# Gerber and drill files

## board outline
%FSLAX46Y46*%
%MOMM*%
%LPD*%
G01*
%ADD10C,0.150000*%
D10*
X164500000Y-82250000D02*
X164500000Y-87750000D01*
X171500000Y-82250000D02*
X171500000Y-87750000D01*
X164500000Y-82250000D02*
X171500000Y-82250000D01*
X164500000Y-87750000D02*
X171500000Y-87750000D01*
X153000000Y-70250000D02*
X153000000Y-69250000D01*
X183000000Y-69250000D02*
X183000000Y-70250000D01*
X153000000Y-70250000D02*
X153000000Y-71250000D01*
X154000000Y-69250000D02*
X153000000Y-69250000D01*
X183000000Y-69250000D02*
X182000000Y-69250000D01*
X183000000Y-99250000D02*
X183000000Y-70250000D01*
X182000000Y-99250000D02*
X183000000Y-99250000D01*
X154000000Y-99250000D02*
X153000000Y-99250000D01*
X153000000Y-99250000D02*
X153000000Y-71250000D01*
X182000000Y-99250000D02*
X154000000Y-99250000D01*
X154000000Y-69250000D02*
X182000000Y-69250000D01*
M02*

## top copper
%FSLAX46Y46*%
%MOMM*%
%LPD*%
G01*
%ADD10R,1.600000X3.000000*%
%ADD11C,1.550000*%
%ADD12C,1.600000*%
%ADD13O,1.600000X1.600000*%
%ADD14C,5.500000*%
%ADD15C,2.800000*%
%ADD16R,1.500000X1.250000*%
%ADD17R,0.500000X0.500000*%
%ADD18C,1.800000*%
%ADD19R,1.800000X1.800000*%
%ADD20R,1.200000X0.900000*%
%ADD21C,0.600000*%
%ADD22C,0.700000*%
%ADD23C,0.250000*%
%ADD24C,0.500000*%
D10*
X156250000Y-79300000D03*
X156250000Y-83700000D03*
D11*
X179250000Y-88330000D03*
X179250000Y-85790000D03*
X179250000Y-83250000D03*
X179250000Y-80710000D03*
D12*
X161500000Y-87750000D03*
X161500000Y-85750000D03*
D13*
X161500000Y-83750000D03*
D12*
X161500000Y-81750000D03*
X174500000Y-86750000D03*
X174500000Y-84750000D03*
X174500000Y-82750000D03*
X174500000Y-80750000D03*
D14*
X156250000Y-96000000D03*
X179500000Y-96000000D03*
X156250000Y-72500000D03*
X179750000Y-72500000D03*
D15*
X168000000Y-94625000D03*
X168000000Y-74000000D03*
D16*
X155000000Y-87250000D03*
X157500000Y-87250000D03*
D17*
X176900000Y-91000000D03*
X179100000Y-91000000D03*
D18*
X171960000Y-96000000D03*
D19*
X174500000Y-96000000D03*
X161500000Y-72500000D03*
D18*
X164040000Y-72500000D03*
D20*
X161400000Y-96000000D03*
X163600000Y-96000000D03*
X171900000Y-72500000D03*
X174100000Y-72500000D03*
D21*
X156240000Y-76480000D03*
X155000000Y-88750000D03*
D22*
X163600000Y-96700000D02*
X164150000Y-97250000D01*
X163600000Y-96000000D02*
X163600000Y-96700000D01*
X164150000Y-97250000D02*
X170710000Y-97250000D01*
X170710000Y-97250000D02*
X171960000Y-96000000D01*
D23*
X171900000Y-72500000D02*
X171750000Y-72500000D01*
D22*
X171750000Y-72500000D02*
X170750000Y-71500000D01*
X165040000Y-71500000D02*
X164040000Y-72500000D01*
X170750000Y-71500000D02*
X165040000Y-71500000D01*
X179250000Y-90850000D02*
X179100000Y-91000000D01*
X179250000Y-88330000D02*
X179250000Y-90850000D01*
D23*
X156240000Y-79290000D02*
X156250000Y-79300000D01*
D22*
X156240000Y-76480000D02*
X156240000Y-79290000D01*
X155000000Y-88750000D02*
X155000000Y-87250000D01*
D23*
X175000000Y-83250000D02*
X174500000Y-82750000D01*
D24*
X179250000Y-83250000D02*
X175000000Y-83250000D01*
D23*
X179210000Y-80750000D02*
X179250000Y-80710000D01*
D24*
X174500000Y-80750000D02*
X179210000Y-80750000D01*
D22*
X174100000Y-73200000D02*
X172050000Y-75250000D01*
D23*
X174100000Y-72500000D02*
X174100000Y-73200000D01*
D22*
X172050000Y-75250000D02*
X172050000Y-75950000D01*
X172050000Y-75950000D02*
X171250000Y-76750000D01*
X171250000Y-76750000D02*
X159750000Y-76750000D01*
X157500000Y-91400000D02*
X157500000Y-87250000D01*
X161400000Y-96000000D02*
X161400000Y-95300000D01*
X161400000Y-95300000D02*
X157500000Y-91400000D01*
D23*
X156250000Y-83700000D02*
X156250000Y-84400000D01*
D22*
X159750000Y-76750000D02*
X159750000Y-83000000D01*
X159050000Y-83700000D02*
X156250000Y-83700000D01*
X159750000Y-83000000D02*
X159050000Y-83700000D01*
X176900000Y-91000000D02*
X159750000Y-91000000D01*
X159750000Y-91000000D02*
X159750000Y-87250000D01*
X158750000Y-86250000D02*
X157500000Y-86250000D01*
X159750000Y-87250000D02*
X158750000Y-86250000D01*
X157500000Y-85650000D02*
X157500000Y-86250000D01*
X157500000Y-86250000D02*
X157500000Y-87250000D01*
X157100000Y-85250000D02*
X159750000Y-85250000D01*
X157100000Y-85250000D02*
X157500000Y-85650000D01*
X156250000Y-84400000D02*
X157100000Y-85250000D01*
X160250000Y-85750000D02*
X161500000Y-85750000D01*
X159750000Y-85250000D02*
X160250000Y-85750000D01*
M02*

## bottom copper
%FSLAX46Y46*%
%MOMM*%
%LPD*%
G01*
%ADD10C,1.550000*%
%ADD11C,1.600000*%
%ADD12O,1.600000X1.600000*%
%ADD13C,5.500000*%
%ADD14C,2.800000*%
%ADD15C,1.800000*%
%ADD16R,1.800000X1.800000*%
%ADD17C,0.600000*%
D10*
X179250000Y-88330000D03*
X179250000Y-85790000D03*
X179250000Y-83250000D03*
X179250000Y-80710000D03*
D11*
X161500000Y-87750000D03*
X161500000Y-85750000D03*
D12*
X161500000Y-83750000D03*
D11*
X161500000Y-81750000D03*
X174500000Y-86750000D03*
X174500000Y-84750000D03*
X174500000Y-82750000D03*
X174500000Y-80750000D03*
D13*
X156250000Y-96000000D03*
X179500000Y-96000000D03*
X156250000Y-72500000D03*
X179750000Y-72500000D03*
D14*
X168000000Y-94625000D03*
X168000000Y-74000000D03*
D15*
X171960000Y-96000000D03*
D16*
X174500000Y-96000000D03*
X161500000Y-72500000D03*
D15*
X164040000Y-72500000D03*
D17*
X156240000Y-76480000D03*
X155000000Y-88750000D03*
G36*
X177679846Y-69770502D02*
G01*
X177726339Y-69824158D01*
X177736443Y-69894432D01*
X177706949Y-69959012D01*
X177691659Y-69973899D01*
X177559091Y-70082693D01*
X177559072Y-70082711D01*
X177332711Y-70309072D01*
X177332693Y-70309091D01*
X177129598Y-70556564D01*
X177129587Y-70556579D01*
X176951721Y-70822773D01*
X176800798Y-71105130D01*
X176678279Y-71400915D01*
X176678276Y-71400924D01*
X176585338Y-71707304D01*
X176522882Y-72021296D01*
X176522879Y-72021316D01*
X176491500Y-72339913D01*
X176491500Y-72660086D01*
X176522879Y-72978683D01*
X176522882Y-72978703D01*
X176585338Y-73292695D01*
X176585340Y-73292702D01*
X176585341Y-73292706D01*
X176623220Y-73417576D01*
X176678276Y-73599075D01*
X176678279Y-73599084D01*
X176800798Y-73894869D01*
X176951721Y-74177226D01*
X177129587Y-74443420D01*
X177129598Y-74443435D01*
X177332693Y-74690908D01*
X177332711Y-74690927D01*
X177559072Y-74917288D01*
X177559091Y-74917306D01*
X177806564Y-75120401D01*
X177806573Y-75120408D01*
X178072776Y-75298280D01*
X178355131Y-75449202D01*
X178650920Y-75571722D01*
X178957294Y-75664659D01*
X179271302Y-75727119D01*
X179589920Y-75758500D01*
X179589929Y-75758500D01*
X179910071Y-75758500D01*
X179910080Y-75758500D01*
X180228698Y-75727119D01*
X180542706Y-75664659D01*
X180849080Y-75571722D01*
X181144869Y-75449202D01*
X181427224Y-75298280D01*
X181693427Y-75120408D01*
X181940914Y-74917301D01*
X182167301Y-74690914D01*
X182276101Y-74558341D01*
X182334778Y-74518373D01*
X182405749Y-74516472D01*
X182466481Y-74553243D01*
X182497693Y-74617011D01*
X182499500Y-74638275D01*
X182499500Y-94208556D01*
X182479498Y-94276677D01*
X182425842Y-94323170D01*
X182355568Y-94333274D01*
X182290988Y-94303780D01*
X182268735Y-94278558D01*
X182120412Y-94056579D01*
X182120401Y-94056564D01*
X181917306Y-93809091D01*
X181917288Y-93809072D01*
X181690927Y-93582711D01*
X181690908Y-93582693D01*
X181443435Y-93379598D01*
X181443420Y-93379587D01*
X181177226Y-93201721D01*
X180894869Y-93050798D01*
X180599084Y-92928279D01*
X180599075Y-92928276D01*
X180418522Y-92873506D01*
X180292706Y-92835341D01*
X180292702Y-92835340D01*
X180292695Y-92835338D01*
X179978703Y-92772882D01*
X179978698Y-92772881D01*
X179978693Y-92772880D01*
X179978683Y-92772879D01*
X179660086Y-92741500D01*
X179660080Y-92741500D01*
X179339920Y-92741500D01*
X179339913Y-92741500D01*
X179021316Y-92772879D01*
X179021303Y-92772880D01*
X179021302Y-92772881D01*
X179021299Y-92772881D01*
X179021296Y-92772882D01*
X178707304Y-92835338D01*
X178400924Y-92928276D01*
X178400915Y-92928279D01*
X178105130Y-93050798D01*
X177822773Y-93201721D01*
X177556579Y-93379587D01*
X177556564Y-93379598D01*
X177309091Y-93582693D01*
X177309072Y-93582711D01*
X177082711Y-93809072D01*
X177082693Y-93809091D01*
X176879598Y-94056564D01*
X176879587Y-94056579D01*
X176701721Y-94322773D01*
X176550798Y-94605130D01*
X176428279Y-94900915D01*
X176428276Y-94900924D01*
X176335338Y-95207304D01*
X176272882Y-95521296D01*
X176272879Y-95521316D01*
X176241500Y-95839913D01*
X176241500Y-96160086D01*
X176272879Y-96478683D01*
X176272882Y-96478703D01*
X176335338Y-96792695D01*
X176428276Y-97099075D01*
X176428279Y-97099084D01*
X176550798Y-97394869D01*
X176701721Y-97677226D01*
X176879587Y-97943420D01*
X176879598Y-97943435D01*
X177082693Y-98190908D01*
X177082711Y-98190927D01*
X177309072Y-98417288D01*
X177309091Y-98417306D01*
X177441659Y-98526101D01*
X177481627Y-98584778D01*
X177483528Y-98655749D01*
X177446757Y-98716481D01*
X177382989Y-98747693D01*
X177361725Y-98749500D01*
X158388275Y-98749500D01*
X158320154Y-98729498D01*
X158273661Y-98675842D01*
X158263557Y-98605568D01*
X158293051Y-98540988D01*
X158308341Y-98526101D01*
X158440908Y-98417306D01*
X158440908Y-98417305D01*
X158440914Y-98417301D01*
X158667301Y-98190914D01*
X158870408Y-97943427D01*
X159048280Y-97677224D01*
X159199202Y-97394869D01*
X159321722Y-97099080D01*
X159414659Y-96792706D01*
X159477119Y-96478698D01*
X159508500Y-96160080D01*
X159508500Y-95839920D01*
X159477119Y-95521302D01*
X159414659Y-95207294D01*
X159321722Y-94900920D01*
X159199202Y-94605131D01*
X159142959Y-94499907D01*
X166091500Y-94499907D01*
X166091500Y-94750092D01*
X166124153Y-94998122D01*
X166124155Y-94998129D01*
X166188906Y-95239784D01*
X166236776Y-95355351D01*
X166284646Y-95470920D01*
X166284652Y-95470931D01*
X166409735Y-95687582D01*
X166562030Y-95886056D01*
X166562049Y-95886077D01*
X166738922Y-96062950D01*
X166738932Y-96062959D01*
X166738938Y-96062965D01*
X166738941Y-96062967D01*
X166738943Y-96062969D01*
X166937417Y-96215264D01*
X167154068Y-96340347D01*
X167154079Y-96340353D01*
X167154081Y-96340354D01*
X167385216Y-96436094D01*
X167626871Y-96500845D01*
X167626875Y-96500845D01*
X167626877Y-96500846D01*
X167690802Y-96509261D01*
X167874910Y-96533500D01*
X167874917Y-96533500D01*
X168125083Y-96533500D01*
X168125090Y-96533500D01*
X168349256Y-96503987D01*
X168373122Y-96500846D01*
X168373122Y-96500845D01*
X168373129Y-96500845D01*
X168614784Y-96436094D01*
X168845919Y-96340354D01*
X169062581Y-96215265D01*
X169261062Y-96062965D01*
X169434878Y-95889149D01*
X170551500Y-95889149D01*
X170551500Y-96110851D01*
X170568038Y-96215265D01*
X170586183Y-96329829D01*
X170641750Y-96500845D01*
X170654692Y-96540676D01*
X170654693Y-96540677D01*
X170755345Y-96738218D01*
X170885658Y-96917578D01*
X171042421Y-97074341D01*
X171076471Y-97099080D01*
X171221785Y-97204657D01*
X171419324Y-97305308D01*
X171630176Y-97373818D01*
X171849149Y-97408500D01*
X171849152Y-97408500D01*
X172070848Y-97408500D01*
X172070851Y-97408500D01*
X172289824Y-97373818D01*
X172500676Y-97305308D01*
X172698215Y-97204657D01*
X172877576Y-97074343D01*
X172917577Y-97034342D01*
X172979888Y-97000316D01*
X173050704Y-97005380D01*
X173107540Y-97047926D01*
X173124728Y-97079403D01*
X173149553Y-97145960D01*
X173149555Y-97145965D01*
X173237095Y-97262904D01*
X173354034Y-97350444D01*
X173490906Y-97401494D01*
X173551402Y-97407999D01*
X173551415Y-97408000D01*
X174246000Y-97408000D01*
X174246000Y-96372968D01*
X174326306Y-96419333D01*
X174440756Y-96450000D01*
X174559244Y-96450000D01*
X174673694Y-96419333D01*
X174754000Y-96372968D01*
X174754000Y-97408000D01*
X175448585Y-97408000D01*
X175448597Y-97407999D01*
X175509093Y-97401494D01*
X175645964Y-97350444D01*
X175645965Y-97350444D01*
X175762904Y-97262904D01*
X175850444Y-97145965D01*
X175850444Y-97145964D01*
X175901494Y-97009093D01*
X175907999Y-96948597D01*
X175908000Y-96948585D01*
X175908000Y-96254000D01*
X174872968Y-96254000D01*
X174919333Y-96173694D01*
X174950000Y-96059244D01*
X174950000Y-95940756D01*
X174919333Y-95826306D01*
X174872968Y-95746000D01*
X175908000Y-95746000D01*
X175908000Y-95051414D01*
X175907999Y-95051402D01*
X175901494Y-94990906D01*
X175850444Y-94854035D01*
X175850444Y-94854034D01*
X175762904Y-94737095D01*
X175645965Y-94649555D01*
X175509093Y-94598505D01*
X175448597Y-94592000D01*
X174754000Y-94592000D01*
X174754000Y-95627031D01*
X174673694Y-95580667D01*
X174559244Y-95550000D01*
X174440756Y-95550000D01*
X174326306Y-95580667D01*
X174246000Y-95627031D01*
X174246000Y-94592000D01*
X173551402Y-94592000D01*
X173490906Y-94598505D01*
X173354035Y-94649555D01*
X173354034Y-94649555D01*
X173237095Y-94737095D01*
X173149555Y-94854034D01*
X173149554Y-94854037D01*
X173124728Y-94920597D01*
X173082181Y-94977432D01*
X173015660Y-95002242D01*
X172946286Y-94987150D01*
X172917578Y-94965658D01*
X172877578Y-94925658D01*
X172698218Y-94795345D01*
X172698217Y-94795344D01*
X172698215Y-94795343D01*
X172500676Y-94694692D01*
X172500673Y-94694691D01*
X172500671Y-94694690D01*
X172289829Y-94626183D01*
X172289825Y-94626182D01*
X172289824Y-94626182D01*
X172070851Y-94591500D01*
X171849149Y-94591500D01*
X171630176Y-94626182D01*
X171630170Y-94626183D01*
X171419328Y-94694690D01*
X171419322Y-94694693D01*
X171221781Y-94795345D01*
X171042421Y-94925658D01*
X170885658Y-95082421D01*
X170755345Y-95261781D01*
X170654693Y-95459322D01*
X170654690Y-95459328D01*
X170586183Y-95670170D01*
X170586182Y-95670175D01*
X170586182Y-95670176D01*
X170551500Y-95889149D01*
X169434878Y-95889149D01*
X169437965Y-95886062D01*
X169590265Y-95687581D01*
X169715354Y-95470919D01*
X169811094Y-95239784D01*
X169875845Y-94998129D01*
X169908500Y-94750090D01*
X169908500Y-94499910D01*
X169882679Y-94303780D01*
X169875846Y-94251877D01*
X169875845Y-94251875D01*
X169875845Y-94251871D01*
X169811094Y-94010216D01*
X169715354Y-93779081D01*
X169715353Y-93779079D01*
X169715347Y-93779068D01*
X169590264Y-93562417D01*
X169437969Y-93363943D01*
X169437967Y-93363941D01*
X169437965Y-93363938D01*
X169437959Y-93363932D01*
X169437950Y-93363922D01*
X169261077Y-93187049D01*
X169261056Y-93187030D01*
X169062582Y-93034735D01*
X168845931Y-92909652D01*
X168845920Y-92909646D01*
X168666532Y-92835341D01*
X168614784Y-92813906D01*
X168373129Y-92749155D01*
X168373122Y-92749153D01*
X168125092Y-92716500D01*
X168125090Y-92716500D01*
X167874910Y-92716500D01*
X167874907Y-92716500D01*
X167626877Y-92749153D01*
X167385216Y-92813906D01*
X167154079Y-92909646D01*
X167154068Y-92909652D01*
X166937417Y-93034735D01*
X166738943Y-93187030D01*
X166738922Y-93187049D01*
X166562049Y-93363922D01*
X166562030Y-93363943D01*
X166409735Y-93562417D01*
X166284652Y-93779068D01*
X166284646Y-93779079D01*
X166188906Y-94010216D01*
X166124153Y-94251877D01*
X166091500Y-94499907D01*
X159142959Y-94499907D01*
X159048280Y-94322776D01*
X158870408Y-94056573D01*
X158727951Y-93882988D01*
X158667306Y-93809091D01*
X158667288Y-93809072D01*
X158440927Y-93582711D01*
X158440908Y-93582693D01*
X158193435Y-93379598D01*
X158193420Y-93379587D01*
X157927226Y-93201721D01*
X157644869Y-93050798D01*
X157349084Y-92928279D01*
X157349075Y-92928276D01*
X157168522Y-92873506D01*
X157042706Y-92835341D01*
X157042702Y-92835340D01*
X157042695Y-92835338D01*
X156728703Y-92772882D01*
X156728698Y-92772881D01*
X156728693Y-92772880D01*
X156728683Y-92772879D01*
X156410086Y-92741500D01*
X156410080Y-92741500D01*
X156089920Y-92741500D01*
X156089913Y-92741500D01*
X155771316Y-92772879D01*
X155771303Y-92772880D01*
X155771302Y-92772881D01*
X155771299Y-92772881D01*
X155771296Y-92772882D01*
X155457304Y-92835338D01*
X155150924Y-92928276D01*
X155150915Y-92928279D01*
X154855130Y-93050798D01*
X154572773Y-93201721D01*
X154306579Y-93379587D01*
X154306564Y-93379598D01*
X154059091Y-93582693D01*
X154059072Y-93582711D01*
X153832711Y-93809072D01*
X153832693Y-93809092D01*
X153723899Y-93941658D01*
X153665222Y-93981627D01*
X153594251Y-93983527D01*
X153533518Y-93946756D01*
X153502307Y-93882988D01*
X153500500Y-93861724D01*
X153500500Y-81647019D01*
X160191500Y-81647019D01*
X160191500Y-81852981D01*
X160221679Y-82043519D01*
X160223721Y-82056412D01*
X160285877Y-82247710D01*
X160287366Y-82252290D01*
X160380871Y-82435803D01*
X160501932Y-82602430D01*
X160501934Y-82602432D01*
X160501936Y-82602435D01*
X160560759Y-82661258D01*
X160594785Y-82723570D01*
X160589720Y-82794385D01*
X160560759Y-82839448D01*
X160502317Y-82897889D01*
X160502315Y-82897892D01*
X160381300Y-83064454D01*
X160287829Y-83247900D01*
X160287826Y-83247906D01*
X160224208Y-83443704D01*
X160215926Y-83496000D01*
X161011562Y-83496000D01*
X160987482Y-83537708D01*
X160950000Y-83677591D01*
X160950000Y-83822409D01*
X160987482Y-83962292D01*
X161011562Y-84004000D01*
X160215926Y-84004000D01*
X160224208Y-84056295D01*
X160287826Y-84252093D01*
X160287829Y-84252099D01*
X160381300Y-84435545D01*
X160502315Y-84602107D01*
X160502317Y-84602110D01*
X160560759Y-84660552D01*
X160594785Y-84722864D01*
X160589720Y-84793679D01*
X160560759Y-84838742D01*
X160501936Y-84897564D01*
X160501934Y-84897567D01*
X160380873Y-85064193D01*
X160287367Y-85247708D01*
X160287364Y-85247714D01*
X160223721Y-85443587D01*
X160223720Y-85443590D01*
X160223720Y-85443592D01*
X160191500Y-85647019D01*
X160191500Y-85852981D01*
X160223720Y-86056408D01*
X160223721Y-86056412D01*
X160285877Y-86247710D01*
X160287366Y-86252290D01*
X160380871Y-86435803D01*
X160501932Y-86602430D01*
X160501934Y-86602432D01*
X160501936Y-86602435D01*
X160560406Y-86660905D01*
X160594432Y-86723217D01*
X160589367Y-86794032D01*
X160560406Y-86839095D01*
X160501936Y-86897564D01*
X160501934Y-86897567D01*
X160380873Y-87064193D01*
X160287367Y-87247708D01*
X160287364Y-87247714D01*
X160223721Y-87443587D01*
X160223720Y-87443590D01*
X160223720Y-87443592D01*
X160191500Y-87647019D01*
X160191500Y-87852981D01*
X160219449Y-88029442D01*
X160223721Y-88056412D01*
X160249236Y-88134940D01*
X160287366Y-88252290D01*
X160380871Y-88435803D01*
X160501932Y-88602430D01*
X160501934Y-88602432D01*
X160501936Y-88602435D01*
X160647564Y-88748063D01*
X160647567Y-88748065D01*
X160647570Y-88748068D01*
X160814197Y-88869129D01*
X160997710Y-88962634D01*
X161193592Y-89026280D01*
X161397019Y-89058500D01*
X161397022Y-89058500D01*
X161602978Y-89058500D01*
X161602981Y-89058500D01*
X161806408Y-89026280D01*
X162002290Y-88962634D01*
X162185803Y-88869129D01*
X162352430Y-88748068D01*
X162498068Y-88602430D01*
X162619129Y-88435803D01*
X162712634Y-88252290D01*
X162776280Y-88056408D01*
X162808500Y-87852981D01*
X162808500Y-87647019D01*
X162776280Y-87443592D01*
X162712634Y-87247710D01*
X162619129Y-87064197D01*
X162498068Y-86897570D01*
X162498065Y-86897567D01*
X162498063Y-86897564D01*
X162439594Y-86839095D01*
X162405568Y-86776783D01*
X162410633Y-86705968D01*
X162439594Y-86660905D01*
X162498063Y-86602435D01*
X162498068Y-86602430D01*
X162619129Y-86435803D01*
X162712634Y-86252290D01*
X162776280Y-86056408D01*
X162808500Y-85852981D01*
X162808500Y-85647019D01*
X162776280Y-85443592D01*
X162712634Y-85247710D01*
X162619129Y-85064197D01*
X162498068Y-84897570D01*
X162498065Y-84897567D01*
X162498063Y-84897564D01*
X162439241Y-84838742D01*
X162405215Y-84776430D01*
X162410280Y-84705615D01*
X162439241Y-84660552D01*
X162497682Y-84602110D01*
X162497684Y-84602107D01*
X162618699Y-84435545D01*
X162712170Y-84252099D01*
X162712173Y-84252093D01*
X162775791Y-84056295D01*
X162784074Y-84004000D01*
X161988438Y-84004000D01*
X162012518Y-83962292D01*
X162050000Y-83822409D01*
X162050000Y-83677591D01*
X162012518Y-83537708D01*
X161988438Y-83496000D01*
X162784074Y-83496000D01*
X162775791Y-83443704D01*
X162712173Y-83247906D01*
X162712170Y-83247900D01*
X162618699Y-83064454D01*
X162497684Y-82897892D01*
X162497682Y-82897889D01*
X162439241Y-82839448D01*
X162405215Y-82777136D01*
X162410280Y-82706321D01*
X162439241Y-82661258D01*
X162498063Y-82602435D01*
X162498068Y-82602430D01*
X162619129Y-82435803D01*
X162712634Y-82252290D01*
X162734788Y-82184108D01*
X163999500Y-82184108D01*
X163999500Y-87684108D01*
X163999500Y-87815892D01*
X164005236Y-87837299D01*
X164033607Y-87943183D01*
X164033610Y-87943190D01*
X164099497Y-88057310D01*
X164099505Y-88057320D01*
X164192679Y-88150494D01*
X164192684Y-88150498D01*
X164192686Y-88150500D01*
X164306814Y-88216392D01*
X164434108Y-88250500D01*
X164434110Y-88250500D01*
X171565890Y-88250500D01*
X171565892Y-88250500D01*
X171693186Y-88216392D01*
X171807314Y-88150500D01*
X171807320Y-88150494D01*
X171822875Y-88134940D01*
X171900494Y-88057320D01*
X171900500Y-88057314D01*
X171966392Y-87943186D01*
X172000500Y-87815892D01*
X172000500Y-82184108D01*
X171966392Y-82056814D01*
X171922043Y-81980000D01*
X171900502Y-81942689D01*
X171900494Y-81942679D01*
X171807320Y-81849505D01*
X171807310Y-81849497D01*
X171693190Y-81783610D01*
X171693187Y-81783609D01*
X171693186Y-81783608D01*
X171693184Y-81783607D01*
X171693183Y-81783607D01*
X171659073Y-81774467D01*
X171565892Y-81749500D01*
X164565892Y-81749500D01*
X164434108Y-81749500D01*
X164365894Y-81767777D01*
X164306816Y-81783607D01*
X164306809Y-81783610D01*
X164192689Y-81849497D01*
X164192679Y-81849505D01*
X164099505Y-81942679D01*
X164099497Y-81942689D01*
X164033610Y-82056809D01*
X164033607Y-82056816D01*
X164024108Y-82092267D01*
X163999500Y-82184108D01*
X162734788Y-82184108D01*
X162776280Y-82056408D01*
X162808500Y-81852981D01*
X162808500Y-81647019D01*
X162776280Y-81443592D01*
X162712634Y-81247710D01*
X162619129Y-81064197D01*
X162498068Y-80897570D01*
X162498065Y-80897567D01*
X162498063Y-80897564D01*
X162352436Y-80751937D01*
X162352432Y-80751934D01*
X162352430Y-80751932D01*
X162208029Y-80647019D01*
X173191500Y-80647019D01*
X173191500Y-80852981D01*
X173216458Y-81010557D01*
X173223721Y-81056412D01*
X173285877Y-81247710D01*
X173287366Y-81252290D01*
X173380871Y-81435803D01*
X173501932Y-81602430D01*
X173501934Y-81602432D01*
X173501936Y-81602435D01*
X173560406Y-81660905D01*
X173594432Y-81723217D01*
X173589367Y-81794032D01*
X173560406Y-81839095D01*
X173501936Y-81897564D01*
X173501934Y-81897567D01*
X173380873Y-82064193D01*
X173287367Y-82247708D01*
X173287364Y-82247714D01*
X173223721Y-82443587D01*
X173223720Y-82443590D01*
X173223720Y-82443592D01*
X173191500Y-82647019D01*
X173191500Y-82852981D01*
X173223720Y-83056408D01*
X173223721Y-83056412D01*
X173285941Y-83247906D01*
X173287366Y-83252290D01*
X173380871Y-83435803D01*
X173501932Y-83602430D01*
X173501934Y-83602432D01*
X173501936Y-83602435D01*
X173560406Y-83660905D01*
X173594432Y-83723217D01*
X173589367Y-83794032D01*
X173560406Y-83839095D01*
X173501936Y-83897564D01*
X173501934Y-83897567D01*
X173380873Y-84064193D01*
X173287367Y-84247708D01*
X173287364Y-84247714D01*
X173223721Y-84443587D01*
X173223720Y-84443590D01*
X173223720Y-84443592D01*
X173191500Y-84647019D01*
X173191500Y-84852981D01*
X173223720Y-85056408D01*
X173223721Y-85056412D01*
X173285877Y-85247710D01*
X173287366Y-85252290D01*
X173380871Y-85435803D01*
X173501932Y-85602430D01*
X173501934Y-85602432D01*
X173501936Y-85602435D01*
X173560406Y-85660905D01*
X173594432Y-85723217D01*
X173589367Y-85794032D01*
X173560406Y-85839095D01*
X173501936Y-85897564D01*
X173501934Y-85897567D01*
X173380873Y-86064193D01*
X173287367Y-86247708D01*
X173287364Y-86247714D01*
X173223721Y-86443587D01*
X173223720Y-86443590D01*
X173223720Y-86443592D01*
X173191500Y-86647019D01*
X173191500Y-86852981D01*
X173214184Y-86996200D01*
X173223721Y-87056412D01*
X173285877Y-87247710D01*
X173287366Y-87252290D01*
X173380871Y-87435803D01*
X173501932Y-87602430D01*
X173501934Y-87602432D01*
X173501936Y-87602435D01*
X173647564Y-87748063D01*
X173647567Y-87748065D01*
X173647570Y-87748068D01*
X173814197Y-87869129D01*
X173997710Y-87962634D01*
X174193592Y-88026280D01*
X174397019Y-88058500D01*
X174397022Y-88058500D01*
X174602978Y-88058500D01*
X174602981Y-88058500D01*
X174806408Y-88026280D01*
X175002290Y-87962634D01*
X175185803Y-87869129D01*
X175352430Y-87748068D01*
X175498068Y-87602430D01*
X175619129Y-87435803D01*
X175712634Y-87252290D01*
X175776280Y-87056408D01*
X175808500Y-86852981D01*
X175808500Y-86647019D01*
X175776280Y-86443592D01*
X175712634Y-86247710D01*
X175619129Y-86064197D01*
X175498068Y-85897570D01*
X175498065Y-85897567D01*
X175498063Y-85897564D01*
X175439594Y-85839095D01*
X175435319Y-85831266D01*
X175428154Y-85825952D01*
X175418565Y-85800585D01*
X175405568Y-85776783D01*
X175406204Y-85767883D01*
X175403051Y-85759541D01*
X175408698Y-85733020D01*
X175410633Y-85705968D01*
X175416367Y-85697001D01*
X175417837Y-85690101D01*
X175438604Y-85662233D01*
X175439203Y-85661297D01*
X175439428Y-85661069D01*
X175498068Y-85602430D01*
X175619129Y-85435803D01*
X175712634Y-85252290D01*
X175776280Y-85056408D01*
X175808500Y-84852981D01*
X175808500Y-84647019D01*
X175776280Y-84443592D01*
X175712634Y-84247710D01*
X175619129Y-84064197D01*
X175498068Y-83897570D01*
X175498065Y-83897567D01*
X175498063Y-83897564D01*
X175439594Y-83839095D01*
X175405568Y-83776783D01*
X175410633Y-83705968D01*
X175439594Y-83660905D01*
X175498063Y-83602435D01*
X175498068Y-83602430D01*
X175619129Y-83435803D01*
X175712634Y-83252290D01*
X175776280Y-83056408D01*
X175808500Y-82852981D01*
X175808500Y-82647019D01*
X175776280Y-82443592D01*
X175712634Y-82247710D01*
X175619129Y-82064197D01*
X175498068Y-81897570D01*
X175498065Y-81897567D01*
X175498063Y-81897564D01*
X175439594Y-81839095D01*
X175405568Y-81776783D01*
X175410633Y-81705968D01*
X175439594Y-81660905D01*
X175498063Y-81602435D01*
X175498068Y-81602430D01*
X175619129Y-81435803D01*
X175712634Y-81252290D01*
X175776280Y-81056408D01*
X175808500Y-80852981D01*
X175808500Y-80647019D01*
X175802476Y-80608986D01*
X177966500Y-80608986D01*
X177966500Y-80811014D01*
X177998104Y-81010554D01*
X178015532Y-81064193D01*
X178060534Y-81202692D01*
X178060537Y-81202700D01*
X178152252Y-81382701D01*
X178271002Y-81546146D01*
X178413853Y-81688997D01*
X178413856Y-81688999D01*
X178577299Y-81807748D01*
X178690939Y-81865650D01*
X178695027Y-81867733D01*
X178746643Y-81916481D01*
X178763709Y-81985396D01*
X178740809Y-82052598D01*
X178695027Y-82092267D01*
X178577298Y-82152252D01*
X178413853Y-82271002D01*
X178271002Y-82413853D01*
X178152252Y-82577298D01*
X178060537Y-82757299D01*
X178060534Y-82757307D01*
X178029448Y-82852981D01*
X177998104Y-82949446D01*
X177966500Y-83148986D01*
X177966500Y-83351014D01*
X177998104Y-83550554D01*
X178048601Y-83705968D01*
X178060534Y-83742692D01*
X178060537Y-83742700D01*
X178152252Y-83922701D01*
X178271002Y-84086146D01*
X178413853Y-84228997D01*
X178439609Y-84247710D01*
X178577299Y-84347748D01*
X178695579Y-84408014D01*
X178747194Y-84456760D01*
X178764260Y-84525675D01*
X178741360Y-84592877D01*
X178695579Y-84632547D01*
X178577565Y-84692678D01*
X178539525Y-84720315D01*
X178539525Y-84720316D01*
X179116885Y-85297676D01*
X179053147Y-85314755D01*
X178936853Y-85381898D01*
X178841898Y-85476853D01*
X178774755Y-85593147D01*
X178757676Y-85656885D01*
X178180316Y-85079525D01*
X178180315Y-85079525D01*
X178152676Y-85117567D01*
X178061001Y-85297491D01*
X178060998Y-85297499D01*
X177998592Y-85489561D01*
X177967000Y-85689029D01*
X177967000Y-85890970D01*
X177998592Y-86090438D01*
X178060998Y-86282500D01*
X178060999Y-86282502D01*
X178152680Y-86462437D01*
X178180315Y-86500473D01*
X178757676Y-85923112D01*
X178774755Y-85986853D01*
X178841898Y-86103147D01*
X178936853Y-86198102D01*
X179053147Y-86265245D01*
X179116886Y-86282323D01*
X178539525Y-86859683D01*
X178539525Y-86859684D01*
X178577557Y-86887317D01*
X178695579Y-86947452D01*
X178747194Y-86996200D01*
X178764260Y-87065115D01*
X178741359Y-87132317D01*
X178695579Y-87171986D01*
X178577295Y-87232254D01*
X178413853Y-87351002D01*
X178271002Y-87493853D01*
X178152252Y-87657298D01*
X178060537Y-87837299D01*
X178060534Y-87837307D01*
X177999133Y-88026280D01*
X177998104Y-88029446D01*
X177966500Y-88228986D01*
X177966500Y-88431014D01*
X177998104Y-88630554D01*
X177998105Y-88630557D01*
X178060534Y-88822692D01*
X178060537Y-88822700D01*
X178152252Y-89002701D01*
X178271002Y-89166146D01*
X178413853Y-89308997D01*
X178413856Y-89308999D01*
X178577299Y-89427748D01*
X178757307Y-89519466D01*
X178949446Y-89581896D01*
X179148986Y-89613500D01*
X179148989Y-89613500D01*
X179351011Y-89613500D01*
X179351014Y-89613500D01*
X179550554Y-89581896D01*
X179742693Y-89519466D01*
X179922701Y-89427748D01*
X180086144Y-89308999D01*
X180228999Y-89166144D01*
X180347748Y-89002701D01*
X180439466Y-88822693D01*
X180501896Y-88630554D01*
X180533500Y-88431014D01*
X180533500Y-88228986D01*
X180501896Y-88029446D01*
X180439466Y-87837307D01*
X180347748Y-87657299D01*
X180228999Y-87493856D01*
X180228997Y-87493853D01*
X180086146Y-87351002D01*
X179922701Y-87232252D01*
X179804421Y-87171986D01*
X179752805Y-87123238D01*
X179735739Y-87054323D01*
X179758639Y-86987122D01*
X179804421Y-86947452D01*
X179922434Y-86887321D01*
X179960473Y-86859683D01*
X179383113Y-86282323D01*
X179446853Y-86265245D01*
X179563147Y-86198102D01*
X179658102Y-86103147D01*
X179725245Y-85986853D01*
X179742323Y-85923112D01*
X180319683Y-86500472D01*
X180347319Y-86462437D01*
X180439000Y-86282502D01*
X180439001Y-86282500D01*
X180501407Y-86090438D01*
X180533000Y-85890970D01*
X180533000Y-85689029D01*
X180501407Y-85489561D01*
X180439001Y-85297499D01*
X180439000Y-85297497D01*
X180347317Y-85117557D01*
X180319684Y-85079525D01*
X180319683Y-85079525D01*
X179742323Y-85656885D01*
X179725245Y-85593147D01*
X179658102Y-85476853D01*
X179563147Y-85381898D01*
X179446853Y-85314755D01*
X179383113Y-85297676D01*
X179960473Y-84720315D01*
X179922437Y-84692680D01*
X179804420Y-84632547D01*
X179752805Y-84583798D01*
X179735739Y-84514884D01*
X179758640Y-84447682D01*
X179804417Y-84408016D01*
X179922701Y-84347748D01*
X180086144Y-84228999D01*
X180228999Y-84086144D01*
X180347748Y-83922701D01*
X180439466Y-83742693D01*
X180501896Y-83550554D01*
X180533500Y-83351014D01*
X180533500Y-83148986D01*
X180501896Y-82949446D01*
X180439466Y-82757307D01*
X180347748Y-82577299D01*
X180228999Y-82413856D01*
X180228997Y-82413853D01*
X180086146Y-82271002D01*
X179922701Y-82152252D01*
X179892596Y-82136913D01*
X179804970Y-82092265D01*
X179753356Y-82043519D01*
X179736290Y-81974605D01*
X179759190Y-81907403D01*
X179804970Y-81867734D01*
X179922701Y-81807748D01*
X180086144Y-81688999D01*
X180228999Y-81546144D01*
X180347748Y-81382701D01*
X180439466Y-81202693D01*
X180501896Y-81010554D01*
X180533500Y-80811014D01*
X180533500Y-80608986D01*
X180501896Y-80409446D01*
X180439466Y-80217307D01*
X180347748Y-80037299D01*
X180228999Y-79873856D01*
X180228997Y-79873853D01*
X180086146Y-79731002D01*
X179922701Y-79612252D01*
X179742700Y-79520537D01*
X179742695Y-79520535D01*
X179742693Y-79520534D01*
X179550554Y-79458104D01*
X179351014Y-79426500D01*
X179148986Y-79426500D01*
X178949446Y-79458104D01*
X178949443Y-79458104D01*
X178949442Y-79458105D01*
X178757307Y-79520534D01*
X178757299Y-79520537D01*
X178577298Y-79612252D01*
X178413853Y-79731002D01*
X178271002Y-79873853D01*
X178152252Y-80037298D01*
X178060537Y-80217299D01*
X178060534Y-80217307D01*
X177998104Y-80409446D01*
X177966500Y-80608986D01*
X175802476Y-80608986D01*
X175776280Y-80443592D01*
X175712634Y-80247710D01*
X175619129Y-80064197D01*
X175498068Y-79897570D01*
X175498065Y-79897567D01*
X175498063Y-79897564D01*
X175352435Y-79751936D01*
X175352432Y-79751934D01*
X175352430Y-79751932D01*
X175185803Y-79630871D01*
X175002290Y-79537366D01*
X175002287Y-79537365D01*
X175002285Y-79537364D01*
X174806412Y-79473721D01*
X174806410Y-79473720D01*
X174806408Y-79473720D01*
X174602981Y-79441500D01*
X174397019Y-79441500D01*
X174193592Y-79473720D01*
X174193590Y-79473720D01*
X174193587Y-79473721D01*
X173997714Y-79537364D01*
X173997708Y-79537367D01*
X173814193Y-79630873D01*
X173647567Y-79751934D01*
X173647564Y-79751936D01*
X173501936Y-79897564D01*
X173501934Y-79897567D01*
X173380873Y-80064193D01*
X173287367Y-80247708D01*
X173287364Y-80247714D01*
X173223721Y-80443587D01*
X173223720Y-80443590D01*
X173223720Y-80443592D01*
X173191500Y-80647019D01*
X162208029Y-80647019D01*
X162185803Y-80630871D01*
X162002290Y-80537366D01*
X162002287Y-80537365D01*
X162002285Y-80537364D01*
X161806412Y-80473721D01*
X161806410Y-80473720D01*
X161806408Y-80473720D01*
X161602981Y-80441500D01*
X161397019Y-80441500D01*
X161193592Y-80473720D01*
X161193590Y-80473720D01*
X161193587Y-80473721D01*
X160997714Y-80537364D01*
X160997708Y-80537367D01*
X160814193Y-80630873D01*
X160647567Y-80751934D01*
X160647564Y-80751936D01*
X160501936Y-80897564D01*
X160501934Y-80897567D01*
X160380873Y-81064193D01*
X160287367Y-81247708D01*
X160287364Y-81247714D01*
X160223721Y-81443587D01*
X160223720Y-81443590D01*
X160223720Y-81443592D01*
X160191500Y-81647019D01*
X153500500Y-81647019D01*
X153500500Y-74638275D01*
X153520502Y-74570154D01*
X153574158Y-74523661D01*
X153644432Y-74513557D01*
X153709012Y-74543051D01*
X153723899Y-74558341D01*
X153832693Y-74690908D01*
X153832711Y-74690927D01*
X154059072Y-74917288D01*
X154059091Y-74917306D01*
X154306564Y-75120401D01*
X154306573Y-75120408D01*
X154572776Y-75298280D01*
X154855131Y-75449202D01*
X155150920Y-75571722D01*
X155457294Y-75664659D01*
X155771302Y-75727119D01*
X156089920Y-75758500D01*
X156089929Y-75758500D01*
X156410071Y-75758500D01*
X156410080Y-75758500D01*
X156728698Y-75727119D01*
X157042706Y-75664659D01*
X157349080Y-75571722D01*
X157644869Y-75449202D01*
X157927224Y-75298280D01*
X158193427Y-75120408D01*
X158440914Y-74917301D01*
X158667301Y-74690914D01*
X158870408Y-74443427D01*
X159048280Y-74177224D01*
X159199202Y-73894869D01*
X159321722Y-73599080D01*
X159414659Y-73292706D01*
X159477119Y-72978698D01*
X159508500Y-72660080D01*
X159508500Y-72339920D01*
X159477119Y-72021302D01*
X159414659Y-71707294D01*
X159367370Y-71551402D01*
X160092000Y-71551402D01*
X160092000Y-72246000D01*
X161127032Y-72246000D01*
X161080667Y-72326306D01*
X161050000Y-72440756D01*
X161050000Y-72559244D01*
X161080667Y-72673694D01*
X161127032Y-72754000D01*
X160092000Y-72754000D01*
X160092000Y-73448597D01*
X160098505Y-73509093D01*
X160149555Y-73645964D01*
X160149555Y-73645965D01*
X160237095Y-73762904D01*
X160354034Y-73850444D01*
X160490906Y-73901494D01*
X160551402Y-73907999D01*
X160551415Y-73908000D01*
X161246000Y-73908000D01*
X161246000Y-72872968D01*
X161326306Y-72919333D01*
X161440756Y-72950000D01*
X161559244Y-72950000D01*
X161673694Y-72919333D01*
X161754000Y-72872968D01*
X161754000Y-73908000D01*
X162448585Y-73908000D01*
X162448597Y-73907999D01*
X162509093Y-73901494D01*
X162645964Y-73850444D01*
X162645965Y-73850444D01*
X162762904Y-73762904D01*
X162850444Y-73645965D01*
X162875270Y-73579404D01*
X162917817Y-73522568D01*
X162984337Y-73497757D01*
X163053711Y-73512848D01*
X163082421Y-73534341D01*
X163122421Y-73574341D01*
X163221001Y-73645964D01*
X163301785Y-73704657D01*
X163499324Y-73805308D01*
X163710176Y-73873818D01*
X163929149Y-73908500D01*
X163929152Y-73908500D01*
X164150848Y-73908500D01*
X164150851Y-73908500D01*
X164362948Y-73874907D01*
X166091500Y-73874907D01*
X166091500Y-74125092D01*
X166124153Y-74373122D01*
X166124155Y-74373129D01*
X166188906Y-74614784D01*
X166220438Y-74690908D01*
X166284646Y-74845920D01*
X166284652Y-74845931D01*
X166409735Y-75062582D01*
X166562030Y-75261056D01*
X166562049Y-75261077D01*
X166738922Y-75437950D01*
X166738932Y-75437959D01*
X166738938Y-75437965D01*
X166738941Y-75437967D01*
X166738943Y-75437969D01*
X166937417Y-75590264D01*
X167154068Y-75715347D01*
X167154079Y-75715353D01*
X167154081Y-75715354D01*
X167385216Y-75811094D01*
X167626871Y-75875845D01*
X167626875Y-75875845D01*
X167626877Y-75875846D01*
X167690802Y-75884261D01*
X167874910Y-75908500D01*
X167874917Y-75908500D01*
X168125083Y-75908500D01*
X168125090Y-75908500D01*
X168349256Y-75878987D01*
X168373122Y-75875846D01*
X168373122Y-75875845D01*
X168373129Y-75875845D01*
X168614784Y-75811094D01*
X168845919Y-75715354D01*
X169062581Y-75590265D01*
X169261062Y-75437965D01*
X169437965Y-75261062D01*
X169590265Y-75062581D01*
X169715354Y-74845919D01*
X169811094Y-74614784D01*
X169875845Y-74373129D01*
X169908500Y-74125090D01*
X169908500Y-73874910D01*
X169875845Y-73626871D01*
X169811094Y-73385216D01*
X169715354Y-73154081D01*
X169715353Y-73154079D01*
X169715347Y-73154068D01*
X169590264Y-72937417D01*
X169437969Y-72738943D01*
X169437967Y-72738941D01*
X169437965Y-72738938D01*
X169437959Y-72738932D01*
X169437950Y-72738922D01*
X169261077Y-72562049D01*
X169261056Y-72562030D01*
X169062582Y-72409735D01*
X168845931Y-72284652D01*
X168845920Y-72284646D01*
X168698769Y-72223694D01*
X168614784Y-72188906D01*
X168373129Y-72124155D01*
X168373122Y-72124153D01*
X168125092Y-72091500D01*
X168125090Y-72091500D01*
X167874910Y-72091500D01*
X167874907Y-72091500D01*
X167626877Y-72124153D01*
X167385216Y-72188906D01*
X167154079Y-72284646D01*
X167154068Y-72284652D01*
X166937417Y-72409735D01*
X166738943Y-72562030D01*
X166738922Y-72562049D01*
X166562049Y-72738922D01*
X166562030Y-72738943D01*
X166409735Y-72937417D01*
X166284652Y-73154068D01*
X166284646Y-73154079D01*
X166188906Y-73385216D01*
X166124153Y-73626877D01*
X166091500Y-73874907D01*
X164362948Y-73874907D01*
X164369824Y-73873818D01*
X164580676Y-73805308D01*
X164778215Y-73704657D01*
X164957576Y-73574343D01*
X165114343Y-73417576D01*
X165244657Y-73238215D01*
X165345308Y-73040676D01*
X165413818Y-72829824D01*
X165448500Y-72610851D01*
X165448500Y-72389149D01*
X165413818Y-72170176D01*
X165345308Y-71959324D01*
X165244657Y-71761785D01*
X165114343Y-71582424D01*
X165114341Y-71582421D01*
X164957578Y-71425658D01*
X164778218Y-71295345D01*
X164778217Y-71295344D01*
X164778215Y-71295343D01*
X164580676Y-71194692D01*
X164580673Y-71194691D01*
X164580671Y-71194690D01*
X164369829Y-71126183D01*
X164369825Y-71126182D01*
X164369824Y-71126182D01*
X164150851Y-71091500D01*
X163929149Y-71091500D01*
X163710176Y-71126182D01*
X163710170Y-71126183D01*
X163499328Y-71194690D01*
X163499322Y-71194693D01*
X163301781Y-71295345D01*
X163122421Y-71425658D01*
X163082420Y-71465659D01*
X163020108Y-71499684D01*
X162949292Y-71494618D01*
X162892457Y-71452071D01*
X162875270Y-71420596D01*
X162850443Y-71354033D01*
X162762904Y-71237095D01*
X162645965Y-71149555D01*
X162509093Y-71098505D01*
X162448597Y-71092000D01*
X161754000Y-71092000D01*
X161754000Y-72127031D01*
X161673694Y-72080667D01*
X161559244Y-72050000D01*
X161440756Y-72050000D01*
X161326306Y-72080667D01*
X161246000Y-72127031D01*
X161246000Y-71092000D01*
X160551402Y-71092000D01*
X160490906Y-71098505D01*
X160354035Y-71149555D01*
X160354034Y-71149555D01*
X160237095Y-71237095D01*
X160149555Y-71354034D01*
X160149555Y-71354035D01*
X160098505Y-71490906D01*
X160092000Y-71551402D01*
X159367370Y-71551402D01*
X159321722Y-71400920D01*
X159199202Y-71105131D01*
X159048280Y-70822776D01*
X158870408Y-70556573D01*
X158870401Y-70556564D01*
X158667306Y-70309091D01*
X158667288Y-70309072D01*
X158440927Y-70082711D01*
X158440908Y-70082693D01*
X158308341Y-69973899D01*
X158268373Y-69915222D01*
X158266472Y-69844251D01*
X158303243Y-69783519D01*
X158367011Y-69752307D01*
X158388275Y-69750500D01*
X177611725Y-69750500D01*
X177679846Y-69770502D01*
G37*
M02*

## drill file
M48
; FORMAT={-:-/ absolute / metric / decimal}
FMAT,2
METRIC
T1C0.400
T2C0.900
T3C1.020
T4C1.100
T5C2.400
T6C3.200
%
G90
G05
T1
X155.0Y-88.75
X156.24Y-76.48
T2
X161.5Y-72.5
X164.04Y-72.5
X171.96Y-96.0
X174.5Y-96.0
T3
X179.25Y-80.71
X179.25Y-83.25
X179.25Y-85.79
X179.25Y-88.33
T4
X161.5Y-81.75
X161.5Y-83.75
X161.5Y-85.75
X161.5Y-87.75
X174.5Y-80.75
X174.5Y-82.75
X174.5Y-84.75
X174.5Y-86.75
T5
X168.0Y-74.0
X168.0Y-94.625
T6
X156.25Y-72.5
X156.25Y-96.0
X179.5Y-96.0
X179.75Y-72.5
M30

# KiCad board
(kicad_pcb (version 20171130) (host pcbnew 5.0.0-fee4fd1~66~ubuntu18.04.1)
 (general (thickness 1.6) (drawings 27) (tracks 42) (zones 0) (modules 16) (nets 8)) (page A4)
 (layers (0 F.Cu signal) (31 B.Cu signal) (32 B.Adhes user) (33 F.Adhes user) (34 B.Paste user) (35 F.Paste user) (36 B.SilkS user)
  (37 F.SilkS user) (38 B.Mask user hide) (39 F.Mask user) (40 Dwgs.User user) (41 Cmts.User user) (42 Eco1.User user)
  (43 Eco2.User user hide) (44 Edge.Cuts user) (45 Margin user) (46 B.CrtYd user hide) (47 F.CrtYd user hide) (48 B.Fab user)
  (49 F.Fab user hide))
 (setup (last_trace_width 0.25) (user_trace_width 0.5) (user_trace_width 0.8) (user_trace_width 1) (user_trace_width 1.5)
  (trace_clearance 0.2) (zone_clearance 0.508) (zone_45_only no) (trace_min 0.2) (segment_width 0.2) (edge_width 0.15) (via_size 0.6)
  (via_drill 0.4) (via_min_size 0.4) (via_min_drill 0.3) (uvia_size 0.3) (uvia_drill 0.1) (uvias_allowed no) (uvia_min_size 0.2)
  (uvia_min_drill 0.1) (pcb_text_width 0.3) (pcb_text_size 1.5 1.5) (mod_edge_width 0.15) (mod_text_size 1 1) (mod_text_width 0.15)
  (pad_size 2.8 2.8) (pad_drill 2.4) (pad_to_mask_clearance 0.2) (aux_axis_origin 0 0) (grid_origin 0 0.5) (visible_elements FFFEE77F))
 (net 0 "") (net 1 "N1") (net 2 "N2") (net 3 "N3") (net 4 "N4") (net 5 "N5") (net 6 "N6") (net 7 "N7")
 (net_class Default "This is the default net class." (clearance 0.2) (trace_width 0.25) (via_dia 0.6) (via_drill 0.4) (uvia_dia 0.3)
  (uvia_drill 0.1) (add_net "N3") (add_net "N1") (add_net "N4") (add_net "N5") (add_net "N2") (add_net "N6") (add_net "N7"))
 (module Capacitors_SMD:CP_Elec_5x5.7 (layer F.Cu) (at 156.25 81.5 90)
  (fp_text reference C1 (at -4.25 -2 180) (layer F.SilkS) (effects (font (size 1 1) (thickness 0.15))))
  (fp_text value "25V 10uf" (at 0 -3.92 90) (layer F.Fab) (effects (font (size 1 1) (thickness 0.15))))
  (pad 2 smd rect (at 2.2 0 270) (size 3 1.6) (layers F.Cu F.Paste F.Mask) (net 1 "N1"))
  (pad 1 smd rect (at -2.2 0 270) (size 3 1.6) (layers F.Cu F.Paste F.Mask) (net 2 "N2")))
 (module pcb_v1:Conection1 (layer F.Cu) (at 179.25 83.25 90)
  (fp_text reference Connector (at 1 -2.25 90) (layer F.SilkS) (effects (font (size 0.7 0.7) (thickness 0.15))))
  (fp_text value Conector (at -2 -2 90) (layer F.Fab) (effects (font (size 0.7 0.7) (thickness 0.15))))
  (pad 1 thru_hole circle (at -5.08 0 90) (size 1.55 1.55) (drill 1.02) (layers *.Cu *.Mask) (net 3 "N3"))
  (pad 2 thru_hole circle (at -2.54 0 90) (size 1.55 1.55) (drill 1.02) (layers *.Cu *.Mask) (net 1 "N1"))
  (pad 3 thru_hole circle (at 0 0 90) (size 1.55 1.55) (drill 1.02) (layers *.Cu *.Mask) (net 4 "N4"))
  (pad 4 thru_hole circle (at 2.54 0 90) (size 1.55 1.55) (drill 1.02) (layers *.Cu *.Mask) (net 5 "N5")))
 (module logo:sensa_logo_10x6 (layer F.Cu) (at 158.5 91)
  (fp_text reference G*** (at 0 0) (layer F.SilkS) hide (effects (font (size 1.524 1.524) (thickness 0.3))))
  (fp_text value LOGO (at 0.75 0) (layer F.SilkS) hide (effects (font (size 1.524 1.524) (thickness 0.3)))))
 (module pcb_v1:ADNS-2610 (layer F.Cu) (at 168 86.75)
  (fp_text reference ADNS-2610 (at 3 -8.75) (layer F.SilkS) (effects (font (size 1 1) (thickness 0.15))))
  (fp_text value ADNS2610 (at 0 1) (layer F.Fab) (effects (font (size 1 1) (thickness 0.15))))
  (pad 8 thru_hole circle (at -6.5 1) (size 1.6 1.6) (drill 1.1) (layers *.Cu *.Mask))
  (pad 7 thru_hole circle (at -6.5 -1) (size 1.6 1.6) (drill 1.1) (layers *.Cu *.Mask) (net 2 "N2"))
  (pad 6 thru_hole oval (at -6.5 -3) (size 1.6 1.6) (drill 1.1) (layers *.Cu *.Mask) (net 1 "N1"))
  (pad 5 thru_hole circle (at -6.5 -5) (size 1.6 1.6) (drill 1.1) (layers *.Cu *.Mask))
  (pad 1 thru_hole circle (at 6.5 0) (size 1.6 1.6) (drill 1.1) (layers *.Cu *.Mask))
  (pad 2 thru_hole circle (at 6.5 -2) (size 1.6 1.6) (drill 1.1) (layers *.Cu *.Mask))
  (pad 3 thru_hole circle (at 6.5 -4) (size 1.6 1.6) (drill 1.1) (layers *.Cu *.Mask) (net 4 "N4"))
  (pad 4 thru_hole circle (at 6.5 -6) (size 1.6 1.6) (drill 1.1) (layers *.Cu *.Mask) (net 5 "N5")))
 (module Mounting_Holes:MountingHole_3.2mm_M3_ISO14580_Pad (layer F.Cu) (at 156.25 96)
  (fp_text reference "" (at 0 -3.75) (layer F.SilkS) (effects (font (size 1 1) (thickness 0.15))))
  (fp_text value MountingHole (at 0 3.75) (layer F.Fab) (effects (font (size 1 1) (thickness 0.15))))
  (pad 1 thru_hole circle (at 0 0) (size 5.5 5.5) (drill 3.2) (layers *.Cu *.Mask)))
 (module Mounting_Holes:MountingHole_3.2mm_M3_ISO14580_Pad (layer F.Cu) (at 179.5 96)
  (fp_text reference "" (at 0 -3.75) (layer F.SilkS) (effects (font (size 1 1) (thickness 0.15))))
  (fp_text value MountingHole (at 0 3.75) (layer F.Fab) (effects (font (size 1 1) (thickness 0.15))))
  (pad 1 thru_hole circle (at 0 0) (size 5.5 5.5) (drill 3.2) (layers *.Cu *.Mask)))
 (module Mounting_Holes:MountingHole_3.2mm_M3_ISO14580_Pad (layer F.Cu) (at 156.25 72.5)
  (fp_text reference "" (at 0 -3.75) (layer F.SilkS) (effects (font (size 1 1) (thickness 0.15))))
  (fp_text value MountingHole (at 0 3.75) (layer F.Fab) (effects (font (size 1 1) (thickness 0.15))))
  (pad 1 thru_hole circle (at 0 0) (size 5.5 5.5) (drill 3.2) (layers *.Cu *.Mask)))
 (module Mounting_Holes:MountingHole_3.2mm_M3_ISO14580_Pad (layer F.Cu) (at 179.75 72.5)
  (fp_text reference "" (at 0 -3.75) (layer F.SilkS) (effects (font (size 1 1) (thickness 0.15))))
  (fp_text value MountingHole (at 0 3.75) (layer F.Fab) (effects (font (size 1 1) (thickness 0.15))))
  (pad 1 thru_hole circle (at 0 0) (size 5.5 5.5) (drill 3.2) (layers *.Cu *.Mask)))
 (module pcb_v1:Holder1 (layer F.Cu) (at 168 81.75)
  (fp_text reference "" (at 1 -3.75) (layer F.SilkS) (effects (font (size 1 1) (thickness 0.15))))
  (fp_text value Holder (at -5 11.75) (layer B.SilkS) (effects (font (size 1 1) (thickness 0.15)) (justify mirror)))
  (pad 1 thru_hole circle (at 0 12.875) (size 2.8 2.8) (drill 2.4) (layers *.Cu *.Mask))
  (pad 2 thru_hole circle (at 0 -7.75) (size 2.8 2.8) (drill 2.4) (layers *.Cu *.Mask)))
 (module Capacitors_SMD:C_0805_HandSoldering (layer F.Cu) (at 156.25 87.25 180)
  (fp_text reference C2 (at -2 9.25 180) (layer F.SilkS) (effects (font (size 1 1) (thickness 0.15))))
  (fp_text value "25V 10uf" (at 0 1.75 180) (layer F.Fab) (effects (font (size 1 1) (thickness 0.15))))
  (pad 2 smd rect (at 1.25 0 180) (size 1.5 1.25) (layers F.Cu F.Paste F.Mask) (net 1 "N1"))
  (pad 1 smd rect (at -1.25 0 180) (size 1.5 1.25) (layers F.Cu F.Paste F.Mask) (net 2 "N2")))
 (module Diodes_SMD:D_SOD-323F (layer F.Cu) (at 178 91 180)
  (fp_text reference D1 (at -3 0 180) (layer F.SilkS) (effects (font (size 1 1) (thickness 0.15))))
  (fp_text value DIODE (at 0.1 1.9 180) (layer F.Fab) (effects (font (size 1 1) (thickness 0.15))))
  (pad 2 smd rect (at 1.1 0 180) (size 0.5 0.5) (layers F.Cu F.Paste F.Mask) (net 2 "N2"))
  (pad 1 smd rect (at -1.1 0 180) (size 0.5 0.5) (layers F.Cu F.Paste F.Mask) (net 3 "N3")))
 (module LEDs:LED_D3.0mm (layer F.Cu) (at 174.5 96 180)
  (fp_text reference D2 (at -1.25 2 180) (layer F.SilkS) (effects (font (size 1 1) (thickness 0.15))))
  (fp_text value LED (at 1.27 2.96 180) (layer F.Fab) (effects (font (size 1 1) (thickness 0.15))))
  (pad 2 thru_hole circle (at 2.54 0 180) (size 1.8 1.8) (drill 0.9) (layers *.Cu *.Mask) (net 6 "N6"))
  (pad 1 thru_hole rect (at 0 0 180) (size 1.8 1.8) (drill 0.9) (layers *.Cu *.Mask) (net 1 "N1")))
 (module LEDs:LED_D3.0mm (layer F.Cu) (at 161.5 72.5)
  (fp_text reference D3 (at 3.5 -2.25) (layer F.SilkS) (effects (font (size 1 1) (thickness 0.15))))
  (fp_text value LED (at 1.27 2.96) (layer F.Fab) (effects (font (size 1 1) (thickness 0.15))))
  (pad 1 thru_hole rect (at 0 0) (size 1.8 1.8) (drill 0.9) (layers *.Cu *.Mask) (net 1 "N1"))
  (pad 2 thru_hole circle (at 2.54 0) (size 1.8 1.8) (drill 0.9) (layers *.Cu *.Mask) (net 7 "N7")))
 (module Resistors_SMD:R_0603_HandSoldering (layer F.Cu) (at 162.5 96 180)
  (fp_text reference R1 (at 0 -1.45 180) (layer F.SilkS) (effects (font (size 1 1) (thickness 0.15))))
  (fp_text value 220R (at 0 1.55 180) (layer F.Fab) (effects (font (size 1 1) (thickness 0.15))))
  (pad 2 smd rect (at 1.1 0 180) (size 1.2 0.9) (layers F.Cu F.Paste F.Mask) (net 2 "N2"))
  (pad 1 smd rect (at -1.1 0 180) (size 1.2 0.9) (layers F.Cu F.Paste F.Mask) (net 6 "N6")))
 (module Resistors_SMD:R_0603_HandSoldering (layer F.Cu) (at 173 72.5)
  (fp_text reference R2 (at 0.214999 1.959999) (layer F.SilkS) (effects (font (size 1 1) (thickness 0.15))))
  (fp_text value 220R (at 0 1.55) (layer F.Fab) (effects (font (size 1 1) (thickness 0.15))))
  (pad 1 smd rect (at -1.1 0) (size 1.2 0.9) (layers F.Cu F.Paste F.Mask) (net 7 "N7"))
  (pad 2 smd rect (at 1.1 0) (size 1.2 0.9) (layers F.Cu F.Paste F.Mask) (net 2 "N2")))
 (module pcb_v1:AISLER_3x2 (layer F.Cu) (at 179.5 77.5)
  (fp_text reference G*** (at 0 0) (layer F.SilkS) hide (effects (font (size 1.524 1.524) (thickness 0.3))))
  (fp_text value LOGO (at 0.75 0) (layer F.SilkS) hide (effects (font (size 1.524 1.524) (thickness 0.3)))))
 (gr_line (start 164.5 82.25) (end 164.5 87.75) (layer Edge.Cuts) (width 0.15))
 (gr_line (start 171.5 82.25) (end 171.5 87.75) (layer Edge.Cuts) (width 0.15))
 (gr_line (start 164.5 82.25) (end 171.5 82.25) (layer Edge.Cuts) (width 0.15))
 (gr_line (start 164.5 87.75) (end 171.5 87.75) (layer Edge.Cuts) (width 0.15))
 (gr_line (start 153 70.25) (end 153 69.25) (layer Edge.Cuts) (width 0.15))
 (gr_line (start 183 69.25) (end 183 70.25) (layer Edge.Cuts) (width 0.15))
 (gr_line (start 153 70.25) (end 153 71.25) (layer Edge.Cuts) (width 0.15))
 (gr_line (start 154 69.25) (end 153 69.25) (layer Edge.Cuts) (width 0.15))
 (gr_line (start 183 69.25) (end 182 69.25) (layer Edge.Cuts) (width 0.15))
 (gr_line (start 183 99.25) (end 183 70.25) (layer Edge.Cuts) (width 0.15))
 (gr_line (start 182 99.25) (end 183 99.25) (layer Edge.Cuts) (width 0.15))
 (gr_line (start 154 99.25) (end 153 99.25) (layer Edge.Cuts) (width 0.15))
 (gr_line (start 153 99.25) (end 153 71.25) (angle 90) (layer Edge.Cuts) (width 0.15))
 (gr_line (start 182 99.25) (end 154 99.25) (angle 90) (layer Edge.Cuts) (width 0.15))
 (gr_line (start 154 69.25) (end 182 69.25) (angle 90) (layer Edge.Cuts) (width 0.15))
 (segment (start 163.6 96.7) (end 164.15 97.25) (width 0.7) (layer F.Cu) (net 6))
 (segment (start 163.6 96) (end 163.6 96.7) (width 0.7) (layer F.Cu) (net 6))
 (segment (start 164.15 97.25) (end 170.71 97.25) (width 0.7) (layer F.Cu) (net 6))
 (segment (start 170.71 97.25) (end 171.96 96) (width 0.7) (layer F.Cu) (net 6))
 (segment (start 171.9 72.5) (end 171.75 72.5) (width 0.25) (layer F.Cu) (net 7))
 (segment (start 171.75 72.5) (end 170.75 71.5) (width 0.7) (layer F.Cu) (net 7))
 (segment (start 165.04 71.5) (end 164.04 72.5) (width 0.7) (layer F.Cu) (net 7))
 (segment (start 170.75 71.5) (end 165.04 71.5) (width 0.7) (layer F.Cu) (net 7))
 (segment (start 179.25 90.85) (end 179.1 91) (width 0.7) (layer F.Cu) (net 3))
 (segment (start 179.25 88.33) (end 179.25 90.85) (width 0.7) (layer F.Cu) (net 3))
 (via (at 156.24 76.48) (size 0.6) (drill 0.4) (layers F.Cu B.Cu) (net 1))
 (via (at 155 88.75) (size 0.6) (drill 0.4) (layers F.Cu B.Cu) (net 1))
 (segment (start 156.24 79.29) (end 156.25 79.3) (width 0.25) (layer F.Cu) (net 1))
 (segment (start 156.24 76.48) (end 156.24 79.29) (width 0.7) (layer F.Cu) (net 1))
 (segment (start 155 88.75) (end 155 87.25) (width 0.7) (layer F.Cu) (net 1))
 (segment (start 175 83.25) (end 174.5 82.75) (width 0.25) (layer F.Cu) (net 4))
 (segment (start 179.25 83.25) (end 175 83.25) (width 0.5) (layer F.Cu) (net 4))
 (segment (start 179.21 80.75) (end 179.25 80.71) (width 0.25) (layer F.Cu) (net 5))
 (segment (start 174.5 80.75) (end 179.21 80.75) (width 0.5) (layer F.Cu) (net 5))
 (segment (start 174.1 73.2) (end 172.05 75.25) (width 0.7) (layer F.Cu) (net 2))
 (segment (start 174.1 72.5) (end 174.1 73.2) (width 0.25) (layer F.Cu) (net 2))
 (segment (start 172.05 75.25) (end 172.05 75.95) (width 0.7) (layer F.Cu) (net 2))
 (segment (start 172.05 75.95) (end 171.25 76.75) (width 0.7) (layer F.Cu) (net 2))
 (segment (start 171.25 76.75) (end 159.75 76.75) (width 0.7) (layer F.Cu) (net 2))
 (segment (start 157.5 91.4) (end 157.5 87.25) (width 0.7) (layer F.Cu) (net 2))
 (segment (start 161.4 96) (end 161.4 95.3) (width 0.7) (layer F.Cu) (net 2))
 (segment (start 161.4 95.3) (end 157.5 91.4) (width 0.7) (layer F.Cu) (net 2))
 (segment (start 156.25 83.7) (end 156.25 84.4) (width 0.25) (layer F.Cu) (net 2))
 (segment (start 159.75 76.75) (end 159.75 83) (width 0.7) (layer F.Cu) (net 2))
 (segment (start 159.05 83.7) (end 156.25 83.7) (width 0.7) (layer F.Cu) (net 2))
 (segment (start 159.75 83) (end 159.05 83.7) (width 0.7) (layer F.Cu) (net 2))
 (segment (start 176.9 91) (end 159.75 91) (width 0.7) (layer F.Cu) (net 2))
 (segment (start 159.75 91) (end 159.75 87.25) (width 0.7) (layer F.Cu) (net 2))
 (segment (start 158.75 86.25) (end 157.5 86.25) (width 0.7) (layer F.Cu) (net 2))
 (segment (start 159.75 87.25) (end 158.75 86.25) (width 0.7) (layer F.Cu) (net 2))
 (segment (start 157.5 85.65) (end 157.5 86.25) (width 0.7) (layer F.Cu) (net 2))
 (segment (start 157.5 86.25) (end 157.5 87.25) (width 0.7) (layer F.Cu) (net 2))
 (segment (start 157.1 85.25) (end 159.75 85.25) (width 0.7) (layer F.Cu) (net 2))
 (segment (start 157.1 85.25) (end 157.5 85.65) (width 0.7) (layer F.Cu) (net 2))
 (segment (start 156.25 84.4) (end 157.1 85.25) (width 0.7) (layer F.Cu) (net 2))
 (segment (start 160.25 85.75) (end 161.5 85.75) (width 0.7) (layer F.Cu) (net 2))
 (segment (start 159.75 85.25) (end 160.25 85.75) (width 0.7) (layer F.Cu) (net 2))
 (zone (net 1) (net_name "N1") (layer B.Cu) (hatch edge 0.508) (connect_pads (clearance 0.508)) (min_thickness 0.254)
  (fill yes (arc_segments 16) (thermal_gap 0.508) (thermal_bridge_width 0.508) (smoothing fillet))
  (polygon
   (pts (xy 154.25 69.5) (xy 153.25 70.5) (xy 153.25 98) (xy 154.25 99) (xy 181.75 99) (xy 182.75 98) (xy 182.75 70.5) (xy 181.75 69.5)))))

